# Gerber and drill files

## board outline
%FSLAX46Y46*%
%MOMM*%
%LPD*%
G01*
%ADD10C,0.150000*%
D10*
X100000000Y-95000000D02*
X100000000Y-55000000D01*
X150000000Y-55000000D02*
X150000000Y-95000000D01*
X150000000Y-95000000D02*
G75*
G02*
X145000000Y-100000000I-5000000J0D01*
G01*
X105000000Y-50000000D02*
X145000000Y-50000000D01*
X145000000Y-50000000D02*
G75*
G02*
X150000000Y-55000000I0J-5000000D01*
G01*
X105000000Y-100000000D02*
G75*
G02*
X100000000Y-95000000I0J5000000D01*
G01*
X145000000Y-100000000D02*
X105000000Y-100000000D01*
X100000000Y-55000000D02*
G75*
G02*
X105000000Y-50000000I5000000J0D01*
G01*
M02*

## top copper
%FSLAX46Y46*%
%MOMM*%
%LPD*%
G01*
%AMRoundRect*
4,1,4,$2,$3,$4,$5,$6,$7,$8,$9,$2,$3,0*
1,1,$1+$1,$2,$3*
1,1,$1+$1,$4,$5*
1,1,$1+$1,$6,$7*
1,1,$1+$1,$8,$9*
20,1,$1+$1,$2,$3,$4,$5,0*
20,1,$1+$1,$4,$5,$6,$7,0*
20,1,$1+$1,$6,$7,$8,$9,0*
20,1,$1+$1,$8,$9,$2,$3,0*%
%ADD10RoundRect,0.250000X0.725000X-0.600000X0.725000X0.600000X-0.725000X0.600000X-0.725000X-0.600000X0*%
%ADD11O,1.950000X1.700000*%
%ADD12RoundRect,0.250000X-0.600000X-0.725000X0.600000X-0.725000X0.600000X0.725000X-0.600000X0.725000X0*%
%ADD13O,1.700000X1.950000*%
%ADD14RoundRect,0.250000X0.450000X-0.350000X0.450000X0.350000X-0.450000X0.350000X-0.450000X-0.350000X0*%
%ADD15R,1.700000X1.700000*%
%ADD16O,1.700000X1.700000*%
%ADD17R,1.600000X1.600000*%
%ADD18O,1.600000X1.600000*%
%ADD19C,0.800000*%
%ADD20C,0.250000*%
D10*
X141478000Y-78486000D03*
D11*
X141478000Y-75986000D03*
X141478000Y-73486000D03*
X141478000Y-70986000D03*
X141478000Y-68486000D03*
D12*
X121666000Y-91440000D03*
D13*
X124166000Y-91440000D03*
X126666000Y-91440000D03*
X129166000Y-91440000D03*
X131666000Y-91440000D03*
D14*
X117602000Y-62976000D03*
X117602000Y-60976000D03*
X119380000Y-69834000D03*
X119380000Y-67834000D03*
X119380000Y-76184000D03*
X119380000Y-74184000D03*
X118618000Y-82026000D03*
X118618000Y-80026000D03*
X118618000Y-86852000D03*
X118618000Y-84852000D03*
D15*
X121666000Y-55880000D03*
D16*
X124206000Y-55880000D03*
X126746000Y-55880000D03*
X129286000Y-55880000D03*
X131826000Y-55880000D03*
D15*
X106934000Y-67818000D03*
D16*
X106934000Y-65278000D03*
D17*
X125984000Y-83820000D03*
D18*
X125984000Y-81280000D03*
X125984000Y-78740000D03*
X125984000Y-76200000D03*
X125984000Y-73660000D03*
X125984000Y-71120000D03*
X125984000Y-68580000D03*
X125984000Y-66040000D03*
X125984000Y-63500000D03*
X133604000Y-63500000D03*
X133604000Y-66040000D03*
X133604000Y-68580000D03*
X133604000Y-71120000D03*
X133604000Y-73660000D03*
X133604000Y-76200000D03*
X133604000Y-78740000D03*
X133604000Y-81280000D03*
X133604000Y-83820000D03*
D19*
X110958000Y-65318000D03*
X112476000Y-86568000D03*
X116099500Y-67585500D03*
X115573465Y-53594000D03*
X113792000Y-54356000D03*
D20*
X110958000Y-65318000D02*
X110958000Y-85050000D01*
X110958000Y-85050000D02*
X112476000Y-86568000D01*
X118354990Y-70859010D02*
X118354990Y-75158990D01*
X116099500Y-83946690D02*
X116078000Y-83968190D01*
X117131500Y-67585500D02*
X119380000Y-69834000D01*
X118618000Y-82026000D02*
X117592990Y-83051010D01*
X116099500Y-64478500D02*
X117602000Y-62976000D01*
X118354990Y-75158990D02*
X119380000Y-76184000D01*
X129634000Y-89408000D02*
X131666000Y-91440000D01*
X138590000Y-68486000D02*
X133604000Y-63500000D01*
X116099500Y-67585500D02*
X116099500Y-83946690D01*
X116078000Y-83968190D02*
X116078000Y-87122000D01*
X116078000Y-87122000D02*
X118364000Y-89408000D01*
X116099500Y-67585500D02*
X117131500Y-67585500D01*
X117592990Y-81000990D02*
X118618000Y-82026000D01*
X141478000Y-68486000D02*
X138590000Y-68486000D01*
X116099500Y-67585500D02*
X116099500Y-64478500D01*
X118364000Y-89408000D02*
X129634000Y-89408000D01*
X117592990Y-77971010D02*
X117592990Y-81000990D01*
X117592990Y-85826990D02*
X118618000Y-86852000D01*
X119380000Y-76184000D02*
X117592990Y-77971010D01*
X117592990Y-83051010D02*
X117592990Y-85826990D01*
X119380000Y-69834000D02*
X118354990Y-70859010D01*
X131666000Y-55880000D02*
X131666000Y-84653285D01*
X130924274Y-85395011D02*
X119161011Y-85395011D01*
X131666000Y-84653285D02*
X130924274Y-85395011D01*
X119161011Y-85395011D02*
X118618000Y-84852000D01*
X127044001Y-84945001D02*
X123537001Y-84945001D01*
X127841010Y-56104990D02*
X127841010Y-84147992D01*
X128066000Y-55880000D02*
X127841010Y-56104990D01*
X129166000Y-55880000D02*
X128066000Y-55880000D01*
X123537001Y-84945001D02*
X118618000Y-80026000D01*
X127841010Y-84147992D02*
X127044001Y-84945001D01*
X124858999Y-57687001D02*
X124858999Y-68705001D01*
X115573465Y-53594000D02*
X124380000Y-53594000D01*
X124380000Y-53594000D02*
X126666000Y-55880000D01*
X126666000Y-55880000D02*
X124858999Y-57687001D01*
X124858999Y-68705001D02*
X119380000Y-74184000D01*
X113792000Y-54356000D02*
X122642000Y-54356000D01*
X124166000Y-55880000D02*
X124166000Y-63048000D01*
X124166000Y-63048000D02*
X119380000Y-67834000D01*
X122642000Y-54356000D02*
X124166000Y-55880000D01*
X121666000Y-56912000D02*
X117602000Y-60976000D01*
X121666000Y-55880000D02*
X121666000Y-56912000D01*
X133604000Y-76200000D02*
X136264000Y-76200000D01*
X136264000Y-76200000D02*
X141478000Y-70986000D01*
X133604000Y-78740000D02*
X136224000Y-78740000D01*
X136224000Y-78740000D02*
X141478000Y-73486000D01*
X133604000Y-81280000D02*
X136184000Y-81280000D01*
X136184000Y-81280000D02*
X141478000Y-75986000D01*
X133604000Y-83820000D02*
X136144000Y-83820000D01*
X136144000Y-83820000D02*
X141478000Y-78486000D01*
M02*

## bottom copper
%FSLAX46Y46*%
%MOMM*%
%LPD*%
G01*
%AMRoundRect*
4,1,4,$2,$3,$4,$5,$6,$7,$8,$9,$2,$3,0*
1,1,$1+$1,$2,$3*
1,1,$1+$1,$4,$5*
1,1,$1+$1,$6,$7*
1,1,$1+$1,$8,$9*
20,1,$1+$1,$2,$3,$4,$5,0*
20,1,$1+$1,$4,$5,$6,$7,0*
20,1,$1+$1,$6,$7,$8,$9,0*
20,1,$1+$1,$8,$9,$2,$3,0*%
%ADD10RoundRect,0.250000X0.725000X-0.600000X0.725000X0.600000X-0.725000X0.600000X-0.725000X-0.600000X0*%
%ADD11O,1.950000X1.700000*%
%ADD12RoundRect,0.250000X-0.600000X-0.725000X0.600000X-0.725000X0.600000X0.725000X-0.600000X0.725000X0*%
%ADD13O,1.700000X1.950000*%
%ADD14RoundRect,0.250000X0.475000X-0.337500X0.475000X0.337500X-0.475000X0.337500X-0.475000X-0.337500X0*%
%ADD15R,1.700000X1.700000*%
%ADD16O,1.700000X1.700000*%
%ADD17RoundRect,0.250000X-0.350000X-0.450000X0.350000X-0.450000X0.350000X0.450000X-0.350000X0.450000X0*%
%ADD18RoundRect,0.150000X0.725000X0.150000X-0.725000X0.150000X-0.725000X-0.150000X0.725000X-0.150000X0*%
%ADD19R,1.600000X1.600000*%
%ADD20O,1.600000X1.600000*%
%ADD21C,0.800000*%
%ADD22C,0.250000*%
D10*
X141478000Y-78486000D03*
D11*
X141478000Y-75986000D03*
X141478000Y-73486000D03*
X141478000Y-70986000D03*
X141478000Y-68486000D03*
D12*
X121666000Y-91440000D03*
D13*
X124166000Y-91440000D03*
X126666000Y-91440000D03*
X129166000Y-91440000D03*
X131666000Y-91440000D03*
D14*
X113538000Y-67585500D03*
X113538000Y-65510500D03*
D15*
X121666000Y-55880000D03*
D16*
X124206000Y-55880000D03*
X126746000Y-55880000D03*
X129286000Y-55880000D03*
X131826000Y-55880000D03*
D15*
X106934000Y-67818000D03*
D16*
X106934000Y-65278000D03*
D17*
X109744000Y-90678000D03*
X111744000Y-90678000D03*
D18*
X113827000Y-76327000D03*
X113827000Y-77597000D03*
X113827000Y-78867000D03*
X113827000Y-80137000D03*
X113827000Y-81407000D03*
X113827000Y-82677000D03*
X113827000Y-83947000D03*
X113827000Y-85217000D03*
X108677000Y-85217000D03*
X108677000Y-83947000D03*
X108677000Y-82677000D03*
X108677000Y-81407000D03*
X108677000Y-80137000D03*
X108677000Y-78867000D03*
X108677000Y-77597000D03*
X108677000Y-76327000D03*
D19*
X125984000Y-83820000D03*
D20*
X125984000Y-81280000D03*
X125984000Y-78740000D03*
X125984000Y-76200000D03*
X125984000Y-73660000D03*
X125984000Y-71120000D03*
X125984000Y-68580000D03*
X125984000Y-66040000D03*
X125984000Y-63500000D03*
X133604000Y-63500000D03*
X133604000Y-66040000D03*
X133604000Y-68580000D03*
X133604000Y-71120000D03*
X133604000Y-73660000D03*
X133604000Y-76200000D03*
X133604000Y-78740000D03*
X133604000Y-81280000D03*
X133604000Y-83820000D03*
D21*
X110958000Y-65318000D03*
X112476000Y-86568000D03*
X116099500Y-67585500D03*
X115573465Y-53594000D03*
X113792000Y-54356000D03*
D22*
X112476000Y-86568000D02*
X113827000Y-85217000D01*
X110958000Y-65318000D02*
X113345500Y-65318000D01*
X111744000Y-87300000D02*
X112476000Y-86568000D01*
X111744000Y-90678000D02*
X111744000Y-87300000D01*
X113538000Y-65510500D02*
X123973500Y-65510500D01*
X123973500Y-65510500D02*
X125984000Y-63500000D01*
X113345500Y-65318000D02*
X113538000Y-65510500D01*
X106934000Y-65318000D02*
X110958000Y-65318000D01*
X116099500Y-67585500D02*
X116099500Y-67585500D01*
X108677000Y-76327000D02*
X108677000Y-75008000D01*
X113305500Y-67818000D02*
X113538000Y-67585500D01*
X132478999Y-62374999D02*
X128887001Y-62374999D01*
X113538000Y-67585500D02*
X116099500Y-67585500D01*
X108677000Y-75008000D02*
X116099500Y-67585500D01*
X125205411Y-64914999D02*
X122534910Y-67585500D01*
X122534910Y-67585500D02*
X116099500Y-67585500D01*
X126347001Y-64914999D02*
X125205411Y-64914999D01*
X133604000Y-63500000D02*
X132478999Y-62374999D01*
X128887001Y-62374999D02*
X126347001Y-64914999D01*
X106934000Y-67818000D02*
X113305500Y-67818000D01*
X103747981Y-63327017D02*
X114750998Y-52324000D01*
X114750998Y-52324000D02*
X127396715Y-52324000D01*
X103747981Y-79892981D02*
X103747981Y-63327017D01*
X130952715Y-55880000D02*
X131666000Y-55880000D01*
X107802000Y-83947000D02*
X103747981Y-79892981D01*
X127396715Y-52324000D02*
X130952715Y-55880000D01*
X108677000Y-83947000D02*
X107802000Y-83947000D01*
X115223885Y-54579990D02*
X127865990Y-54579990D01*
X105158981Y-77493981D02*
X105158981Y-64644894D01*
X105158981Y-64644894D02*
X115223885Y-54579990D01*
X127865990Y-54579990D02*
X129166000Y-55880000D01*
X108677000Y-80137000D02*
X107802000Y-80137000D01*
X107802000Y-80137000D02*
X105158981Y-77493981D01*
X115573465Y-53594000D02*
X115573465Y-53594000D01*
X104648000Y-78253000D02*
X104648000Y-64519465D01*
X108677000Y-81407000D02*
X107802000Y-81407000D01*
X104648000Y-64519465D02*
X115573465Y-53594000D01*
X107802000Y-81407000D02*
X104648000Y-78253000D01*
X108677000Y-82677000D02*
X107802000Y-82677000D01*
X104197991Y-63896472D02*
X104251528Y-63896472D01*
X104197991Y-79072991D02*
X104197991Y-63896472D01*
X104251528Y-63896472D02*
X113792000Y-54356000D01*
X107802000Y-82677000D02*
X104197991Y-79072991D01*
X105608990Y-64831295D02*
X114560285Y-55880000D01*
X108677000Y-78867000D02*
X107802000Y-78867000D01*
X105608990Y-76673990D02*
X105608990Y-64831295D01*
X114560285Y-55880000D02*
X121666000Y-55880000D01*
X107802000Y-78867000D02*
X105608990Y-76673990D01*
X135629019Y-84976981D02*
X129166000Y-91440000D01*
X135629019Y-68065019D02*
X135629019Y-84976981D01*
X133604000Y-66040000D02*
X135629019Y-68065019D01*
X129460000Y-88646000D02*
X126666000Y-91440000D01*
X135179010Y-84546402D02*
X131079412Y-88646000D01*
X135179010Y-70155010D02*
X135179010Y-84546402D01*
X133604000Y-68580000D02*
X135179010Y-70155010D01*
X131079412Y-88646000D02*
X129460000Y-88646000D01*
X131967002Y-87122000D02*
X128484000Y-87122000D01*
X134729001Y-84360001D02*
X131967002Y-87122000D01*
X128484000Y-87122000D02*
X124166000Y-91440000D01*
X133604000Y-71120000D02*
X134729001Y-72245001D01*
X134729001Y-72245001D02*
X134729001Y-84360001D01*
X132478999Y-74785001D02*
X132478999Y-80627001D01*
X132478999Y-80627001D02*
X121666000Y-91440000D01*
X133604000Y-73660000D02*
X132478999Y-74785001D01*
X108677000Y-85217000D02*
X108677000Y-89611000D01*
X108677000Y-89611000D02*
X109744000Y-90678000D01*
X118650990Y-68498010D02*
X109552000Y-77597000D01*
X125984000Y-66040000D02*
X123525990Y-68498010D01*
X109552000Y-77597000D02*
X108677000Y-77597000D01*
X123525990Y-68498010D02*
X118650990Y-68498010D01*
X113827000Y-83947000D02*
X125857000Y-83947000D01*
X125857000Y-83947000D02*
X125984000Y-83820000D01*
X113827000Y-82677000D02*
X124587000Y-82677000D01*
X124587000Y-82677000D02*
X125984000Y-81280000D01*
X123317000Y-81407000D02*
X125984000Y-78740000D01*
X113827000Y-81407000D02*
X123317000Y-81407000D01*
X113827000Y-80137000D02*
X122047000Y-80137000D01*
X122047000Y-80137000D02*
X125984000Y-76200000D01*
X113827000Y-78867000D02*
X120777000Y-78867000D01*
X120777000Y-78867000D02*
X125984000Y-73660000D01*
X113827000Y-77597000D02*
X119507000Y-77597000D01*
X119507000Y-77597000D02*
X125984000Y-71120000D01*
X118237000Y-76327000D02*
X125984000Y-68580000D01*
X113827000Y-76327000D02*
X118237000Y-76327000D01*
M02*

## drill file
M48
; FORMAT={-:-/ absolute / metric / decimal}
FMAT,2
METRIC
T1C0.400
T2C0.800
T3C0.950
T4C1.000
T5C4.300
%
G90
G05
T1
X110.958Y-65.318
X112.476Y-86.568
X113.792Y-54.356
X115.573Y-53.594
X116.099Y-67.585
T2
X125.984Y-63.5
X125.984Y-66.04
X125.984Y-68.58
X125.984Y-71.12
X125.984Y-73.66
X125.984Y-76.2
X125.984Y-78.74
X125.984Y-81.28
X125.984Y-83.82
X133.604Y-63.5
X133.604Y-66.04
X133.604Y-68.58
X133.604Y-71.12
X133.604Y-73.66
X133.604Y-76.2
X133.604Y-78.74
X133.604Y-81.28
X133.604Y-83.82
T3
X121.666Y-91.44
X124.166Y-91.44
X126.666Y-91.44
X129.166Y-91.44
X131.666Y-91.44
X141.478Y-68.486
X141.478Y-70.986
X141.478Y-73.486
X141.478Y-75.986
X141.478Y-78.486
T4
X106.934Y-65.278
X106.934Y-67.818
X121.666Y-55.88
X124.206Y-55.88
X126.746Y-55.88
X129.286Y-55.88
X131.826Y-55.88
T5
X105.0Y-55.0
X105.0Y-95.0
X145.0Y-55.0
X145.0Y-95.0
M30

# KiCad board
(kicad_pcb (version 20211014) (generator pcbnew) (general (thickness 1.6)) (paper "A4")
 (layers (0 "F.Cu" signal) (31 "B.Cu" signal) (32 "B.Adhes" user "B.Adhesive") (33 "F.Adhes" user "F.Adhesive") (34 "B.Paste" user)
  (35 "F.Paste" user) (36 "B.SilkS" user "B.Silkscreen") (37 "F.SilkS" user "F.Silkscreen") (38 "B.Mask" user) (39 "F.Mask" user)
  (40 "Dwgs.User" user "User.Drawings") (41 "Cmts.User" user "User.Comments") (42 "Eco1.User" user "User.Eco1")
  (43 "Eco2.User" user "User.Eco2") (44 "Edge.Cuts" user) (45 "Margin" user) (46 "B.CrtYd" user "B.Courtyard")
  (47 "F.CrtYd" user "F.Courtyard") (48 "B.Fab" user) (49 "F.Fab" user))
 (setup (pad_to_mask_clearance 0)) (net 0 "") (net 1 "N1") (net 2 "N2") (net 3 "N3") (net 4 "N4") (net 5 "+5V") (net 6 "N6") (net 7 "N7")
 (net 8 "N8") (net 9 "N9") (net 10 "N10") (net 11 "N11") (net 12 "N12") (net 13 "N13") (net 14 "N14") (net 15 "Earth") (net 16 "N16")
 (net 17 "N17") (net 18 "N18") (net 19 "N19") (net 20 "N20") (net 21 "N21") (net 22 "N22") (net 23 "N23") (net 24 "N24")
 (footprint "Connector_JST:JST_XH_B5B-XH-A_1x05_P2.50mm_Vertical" (layer "F.Cu") (at 141.478 78.486 90)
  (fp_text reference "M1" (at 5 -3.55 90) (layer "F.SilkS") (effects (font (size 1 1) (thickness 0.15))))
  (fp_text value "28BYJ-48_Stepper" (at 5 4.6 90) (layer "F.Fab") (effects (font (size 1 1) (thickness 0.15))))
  (pad "1" thru_hole roundrect locked (at 0 0 90) (size 1.7 1.95) (drill 0.95) (layers *.Cu *.Mask) (roundrect_rratio 0.1470588235)
   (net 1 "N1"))
  (pad "2" thru_hole oval locked (at 2.5 0 90) (size 1.7 1.95) (drill 0.95) (layers *.Cu *.Mask) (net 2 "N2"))
  (pad "3" thru_hole oval locked (at 5 0 90) (size 1.7 1.95) (drill 0.95) (layers *.Cu *.Mask) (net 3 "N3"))
  (pad "4" thru_hole oval locked (at 7.5 0 90) (size 1.7 1.95) (drill 0.95) (layers *.Cu *.Mask) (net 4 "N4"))
  (pad "5" thru_hole oval locked (at 10 0 90) (size 1.7 1.95) (drill 0.95) (layers *.Cu *.Mask) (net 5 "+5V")))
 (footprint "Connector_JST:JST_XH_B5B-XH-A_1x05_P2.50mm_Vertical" (layer "F.Cu") (at 121.666 91.44)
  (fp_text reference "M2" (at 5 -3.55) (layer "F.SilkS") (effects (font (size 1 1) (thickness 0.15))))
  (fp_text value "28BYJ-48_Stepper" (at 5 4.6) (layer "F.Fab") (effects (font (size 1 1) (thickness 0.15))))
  (pad "1" thru_hole roundrect locked (at 0 0) (size 1.7 1.95) (drill 0.95) (layers *.Cu *.Mask) (roundrect_rratio 0.1470588235)
   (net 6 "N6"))
  (pad "2" thru_hole oval locked (at 2.5 0) (size 1.7 1.95) (drill 0.95) (layers *.Cu *.Mask) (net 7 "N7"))
  (pad "3" thru_hole oval locked (at 5 0) (size 1.7 1.95) (drill 0.95) (layers *.Cu *.Mask) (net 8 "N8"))
  (pad "4" thru_hole oval locked (at 7.5 0) (size 1.7 1.95) (drill 0.95) (layers *.Cu *.Mask) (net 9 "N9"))
  (pad "5" thru_hole oval locked (at 10 0) (size 1.7 1.95) (drill 0.95) (layers *.Cu *.Mask) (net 5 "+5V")))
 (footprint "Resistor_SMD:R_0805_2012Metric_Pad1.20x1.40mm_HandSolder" (layer "F.Cu") (at 117.602 61.976 90)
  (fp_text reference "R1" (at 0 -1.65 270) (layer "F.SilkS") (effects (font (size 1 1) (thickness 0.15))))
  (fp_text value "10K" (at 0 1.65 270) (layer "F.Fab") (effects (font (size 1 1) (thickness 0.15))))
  (pad "1" smd roundrect locked (at -1 0 90) (size 1.2 1.4) (layers "F.Cu" "F.Paste" "F.Mask") (roundrect_rratio 0.2083333333) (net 5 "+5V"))
  (pad "2" smd roundrect locked (at 1 0 90) (size 1.2 1.4) (layers "F.Cu" "F.Paste" "F.Mask") (roundrect_rratio 0.2083333333) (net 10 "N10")))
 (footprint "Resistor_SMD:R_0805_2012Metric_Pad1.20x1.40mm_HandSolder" (layer "F.Cu") (at 119.38 68.834 90)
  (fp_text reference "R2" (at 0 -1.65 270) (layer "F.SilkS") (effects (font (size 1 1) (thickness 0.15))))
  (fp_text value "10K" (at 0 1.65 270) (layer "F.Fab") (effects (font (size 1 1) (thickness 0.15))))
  (pad "1" smd roundrect locked (at -1 0 90) (size 1.2 1.4) (layers "F.Cu" "F.Paste" "F.Mask") (roundrect_rratio 0.2083333333) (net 5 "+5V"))
  (pad "2" smd roundrect locked (at 1 0 90) (size 1.2 1.4) (layers "F.Cu" "F.Paste" "F.Mask") (roundrect_rratio 0.2083333333) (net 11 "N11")))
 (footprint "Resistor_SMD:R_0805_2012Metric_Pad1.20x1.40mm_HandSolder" (layer "F.Cu") (at 119.38 75.184 90)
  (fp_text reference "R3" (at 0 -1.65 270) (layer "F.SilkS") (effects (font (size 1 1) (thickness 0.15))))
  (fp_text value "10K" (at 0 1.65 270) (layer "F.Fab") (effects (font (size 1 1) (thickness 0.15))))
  (pad "1" smd roundrect locked (at -1 0 90) (size 1.2 1.4) (layers "F.Cu" "F.Paste" "F.Mask") (roundrect_rratio 0.2083333333) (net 5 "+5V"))
  (pad "2" smd roundrect locked (at 1 0 90) (size 1.2 1.4) (layers "F.Cu" "F.Paste" "F.Mask") (roundrect_rratio 0.2083333333) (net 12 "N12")))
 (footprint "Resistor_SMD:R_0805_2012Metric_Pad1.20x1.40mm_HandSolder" (layer "F.Cu") (at 118.618 81.026 90)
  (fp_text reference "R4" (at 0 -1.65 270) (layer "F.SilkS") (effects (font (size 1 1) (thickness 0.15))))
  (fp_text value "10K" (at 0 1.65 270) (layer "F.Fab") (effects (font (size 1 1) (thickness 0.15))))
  (pad "1" smd roundrect locked (at -1 0 90) (size 1.2 1.4) (layers "F.Cu" "F.Paste" "F.Mask") (roundrect_rratio 0.2083333333) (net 5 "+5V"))
  (pad "2" smd roundrect locked (at 1 0 90) (size 1.2 1.4) (layers "F.Cu" "F.Paste" "F.Mask") (roundrect_rratio 0.2083333333) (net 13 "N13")))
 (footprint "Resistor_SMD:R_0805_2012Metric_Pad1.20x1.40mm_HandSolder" (layer "F.Cu") (at 118.618 85.852 90)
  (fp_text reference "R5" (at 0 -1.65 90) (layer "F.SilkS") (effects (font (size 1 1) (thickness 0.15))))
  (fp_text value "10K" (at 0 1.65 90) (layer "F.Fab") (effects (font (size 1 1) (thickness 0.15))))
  (pad "1" smd roundrect locked (at -1 0 90) (size 1.2 1.4) (layers "F.Cu" "F.Paste" "F.Mask") (roundrect_rratio 0.2083333333) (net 5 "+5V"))
  (pad "2" smd roundrect locked (at 1 0 90) (size 1.2 1.4) (layers "F.Cu" "F.Paste" "F.Mask") (roundrect_rratio 0.2083333333) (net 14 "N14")))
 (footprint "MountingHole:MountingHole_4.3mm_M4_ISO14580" (layer "F.Cu") (at 105 55)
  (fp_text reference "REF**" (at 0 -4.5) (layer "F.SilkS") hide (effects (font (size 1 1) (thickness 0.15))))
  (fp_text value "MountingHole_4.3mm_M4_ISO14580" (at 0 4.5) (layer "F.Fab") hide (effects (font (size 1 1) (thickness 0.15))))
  (pad "" np_thru_hole circle locked (at 0 0) (size 4.3 4.3) (drill 4.3) (layers *.Cu *.Mask)))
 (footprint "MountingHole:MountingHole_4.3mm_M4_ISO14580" (layer "F.Cu") (at 145 55)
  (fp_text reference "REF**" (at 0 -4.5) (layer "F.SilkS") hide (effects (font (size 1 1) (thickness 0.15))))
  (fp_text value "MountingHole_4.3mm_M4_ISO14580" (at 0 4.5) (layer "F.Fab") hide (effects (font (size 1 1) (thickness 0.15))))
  (pad "" np_thru_hole circle locked (at 0 0) (size 4.3 4.3) (drill 4.3) (layers *.Cu *.Mask)))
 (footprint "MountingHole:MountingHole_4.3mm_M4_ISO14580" (layer "F.Cu") (at 105 95)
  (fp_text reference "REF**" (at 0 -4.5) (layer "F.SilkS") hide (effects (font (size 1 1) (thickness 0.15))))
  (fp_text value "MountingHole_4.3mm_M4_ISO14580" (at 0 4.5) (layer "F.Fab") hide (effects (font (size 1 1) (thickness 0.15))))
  (pad "" np_thru_hole circle locked (at 0 0) (size 4.3 4.3) (drill 4.3) (layers *.Cu *.Mask)))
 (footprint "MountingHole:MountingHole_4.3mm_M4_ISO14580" (layer "F.Cu") (at 145 95)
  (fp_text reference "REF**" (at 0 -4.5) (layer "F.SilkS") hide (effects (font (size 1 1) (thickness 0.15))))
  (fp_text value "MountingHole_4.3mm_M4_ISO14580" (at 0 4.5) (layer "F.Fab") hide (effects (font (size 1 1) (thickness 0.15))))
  (pad "" np_thru_hole circle locked (at 0 0) (size 4.3 4.3) (drill 4.3) (layers *.Cu *.Mask)))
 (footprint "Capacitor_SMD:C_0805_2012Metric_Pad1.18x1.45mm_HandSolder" (layer "B.Cu") (at 113.538 66.548 90)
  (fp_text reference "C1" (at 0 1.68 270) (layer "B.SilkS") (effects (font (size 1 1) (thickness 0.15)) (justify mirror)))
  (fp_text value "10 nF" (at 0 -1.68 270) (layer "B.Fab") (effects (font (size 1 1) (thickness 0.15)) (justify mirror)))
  (pad "1" smd roundrect locked (at -1.0375 0 90) (size 1.175 1.45) (layers "B.Cu" "B.Paste" "B.Mask") (roundrect_rratio 0.2127659574)
   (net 5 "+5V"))
  (pad "2" smd roundrect locked (at 1.0375 0 90) (size 1.175 1.45) (layers "B.Cu" "B.Paste" "B.Mask") (roundrect_rratio 0.2127659574)
   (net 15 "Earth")))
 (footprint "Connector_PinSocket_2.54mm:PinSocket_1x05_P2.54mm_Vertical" (layer "B.Cu") (at 121.666 55.88 -90)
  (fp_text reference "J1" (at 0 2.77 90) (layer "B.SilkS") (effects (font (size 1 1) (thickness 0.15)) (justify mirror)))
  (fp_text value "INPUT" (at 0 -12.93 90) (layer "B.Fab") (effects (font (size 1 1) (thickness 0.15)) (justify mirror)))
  (pad "1" thru_hole rect (at 0 0 270) (size 1.7 1.7) (drill 1) (layers *.Cu *.Mask) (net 10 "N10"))
  (pad "2" thru_hole oval (at 0 -2.54 270) (size 1.7 1.7) (drill 1) (layers *.Cu *.Mask) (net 11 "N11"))
  (pad "3" thru_hole oval (at 0 -5.08 270) (size 1.7 1.7) (drill 1) (layers *.Cu *.Mask) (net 12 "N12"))
  (pad "4" thru_hole oval (at 0 -7.62 270) (size 1.7 1.7) (drill 1) (layers *.Cu *.Mask) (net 13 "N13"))
  (pad "5" thru_hole oval (at 0 -10.16 270) (size 1.7 1.7) (drill 1) (layers *.Cu *.Mask) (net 14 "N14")))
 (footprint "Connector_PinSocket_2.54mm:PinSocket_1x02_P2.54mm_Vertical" (layer "B.Cu") (at 106.934 67.818)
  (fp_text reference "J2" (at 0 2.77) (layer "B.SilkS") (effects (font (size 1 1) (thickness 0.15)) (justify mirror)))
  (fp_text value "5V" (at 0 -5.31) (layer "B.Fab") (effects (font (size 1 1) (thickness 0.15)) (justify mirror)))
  (pad "1" thru_hole rect (at 0 0) (size 1.7 1.7) (drill 1) (layers *.Cu *.Mask) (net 5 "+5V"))
  (pad "2" thru_hole oval (at 0 -2.54) (size 1.7 1.7) (drill 1) (layers *.Cu *.Mask) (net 15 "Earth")))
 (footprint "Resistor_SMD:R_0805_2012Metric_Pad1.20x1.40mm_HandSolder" (layer "B.Cu") (at 110.744 90.678)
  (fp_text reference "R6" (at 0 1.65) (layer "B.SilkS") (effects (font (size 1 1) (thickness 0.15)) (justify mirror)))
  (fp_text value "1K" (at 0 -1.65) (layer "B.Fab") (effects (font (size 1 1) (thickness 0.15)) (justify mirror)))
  (pad "1" smd roundrect locked (at -1 0) (size 1.2 1.4) (layers "B.Cu" "B.Paste" "B.Mask") (roundrect_rratio 0.2083333333) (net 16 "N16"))
  (pad "2" smd roundrect locked (at 1 0) (size 1.2 1.4) (layers "B.Cu" "B.Paste" "B.Mask") (roundrect_rratio 0.2083333333) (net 15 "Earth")))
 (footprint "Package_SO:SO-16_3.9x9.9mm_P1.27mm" (layer "B.Cu") (at 111.252 80.772 180)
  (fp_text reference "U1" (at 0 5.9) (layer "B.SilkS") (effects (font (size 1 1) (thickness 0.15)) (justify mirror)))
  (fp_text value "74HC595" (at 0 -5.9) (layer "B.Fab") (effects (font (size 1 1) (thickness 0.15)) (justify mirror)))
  (pad "1" smd roundrect locked (at -2.575 4.445 180) (size 1.75 0.6) (layers "B.Cu" "B.Paste" "B.Mask") (roundrect_rratio 0.25)
   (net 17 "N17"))
  (pad "2" smd roundrect locked (at -2.575 3.175 180) (size 1.75 0.6) (layers "B.Cu" "B.Paste" "B.Mask") (roundrect_rratio 0.25)
   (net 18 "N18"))
  (pad "3" smd roundrect locked (at -2.575 1.905 180) (size 1.75 0.6) (layers "B.Cu" "B.Paste" "B.Mask") (roundrect_rratio 0.25)
   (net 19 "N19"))
  (pad "4" smd roundrect locked (at -2.575 0.635 180) (size 1.75 0.6) (layers "B.Cu" "B.Paste" "B.Mask") (roundrect_rratio 0.25)
   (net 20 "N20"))
  (pad "5" smd roundrect locked (at -2.575 -0.635 180) (size 1.75 0.6) (layers "B.Cu" "B.Paste" "B.Mask") (roundrect_rratio 0.25)
   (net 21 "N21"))
  (pad "6" smd roundrect locked (at -2.575 -1.905 180) (size 1.75 0.6) (layers "B.Cu" "B.Paste" "B.Mask") (roundrect_rratio 0.25)
   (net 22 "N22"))
  (pad "7" smd roundrect locked (at -2.575 -3.175 180) (size 1.75 0.6) (layers "B.Cu" "B.Paste" "B.Mask") (roundrect_rratio 0.25)
   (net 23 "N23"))
  (pad "8" smd roundrect locked (at -2.575 -4.445 180) (size 1.75 0.6) (layers "B.Cu" "B.Paste" "B.Mask") (roundrect_rratio 0.25)
   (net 15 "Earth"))
  (pad "9" smd roundrect locked (at 2.575 -4.445 180) (size 1.75 0.6) (layers "B.Cu" "B.Paste" "B.Mask") (roundrect_rratio 0.25)
   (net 16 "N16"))
  (pad "10" smd roundrect locked (at 2.575 -3.175 180) (size 1.75 0.6) (layers "B.Cu" "B.Paste" "B.Mask") (roundrect_rratio 0.25)
   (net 14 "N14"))
  (pad "11" smd roundrect locked (at 2.575 -1.905 180) (size 1.75 0.6) (layers "B.Cu" "B.Paste" "B.Mask") (roundrect_rratio 0.25)
   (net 11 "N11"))
  (pad "12" smd roundrect locked (at 2.575 -0.635 180) (size 1.75 0.6) (layers "B.Cu" "B.Paste" "B.Mask") (roundrect_rratio 0.25)
   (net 12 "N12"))
  (pad "13" smd roundrect locked (at 2.575 0.635 180) (size 1.75 0.6) (layers "B.Cu" "B.Paste" "B.Mask") (roundrect_rratio 0.25)
   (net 13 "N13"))
  (pad "14" smd roundrect locked (at 2.575 1.905 180) (size 1.75 0.6) (layers "B.Cu" "B.Paste" "B.Mask") (roundrect_rratio 0.25)
   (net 10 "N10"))
  (pad "15" smd roundrect locked (at 2.575 3.175 180) (size 1.75 0.6) (layers "B.Cu" "B.Paste" "B.Mask") (roundrect_rratio 0.25)
   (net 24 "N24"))
  (pad "16" smd roundrect locked (at 2.575 4.445 180) (size 1.75 0.6) (layers "B.Cu" "B.Paste" "B.Mask") (roundrect_rratio 0.25)
   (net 5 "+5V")))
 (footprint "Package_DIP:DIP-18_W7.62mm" (layer "B.Cu") (at 125.984 83.82)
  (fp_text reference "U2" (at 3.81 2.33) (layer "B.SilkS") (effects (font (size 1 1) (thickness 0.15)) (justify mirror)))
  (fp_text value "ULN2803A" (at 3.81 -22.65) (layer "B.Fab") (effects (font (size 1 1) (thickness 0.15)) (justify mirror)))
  (pad "1" thru_hole rect locked (at 0 0) (size 1.6 1.6) (drill 0.8) (layers *.Cu *.Mask) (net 23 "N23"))
  (pad "2" thru_hole oval locked (at 0 -2.54) (size 1.6 1.6) (drill 0.8) (layers *.Cu *.Mask) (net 22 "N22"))
  (pad "3" thru_hole oval locked (at 0 -5.08) (size 1.6 1.6) (drill 0.8) (layers *.Cu *.Mask) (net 21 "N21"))
  (pad "4" thru_hole oval locked (at 0 -7.62) (size 1.6 1.6) (drill 0.8) (layers *.Cu *.Mask) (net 20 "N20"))
  (pad "5" thru_hole oval locked (at 0 -10.16) (size 1.6 1.6) (drill 0.8) (layers *.Cu *.Mask) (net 19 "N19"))
  (pad "6" thru_hole oval locked (at 0 -12.7) (size 1.6 1.6) (drill 0.8) (layers *.Cu *.Mask) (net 18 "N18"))
  (pad "7" thru_hole oval locked (at 0 -15.24) (size 1.6 1.6) (drill 0.8) (layers *.Cu *.Mask) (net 17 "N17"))
  (pad "8" thru_hole oval locked (at 0 -17.78) (size 1.6 1.6) (drill 0.8) (layers *.Cu *.Mask) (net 24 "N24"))
  (pad "9" thru_hole oval locked (at 0 -20.32) (size 1.6 1.6) (drill 0.8) (layers *.Cu *.Mask) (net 15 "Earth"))
  (pad "10" thru_hole oval locked (at 7.62 -20.32) (size 1.6 1.6) (drill 0.8) (layers *.Cu *.Mask) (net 5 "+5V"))
  (pad "11" thru_hole oval locked (at 7.62 -17.78) (size 1.6 1.6) (drill 0.8) (layers *.Cu *.Mask) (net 9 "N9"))
  (pad "12" thru_hole oval locked (at 7.62 -15.24) (size 1.6 1.6) (drill 0.8) (layers *.Cu *.Mask) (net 8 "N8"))
  (pad "13" thru_hole oval locked (at 7.62 -12.7) (size 1.6 1.6) (drill 0.8) (layers *.Cu *.Mask) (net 7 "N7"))
  (pad "14" thru_hole oval locked (at 7.62 -10.16) (size 1.6 1.6) (drill 0.8) (layers *.Cu *.Mask) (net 6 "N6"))
  (pad "15" thru_hole oval locked (at 7.62 -7.62) (size 1.6 1.6) (drill 0.8) (layers *.Cu *.Mask) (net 4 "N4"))
  (pad "16" thru_hole oval locked (at 7.62 -5.08) (size 1.6 1.6) (drill 0.8) (layers *.Cu *.Mask) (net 3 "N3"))
  (pad "17" thru_hole oval locked (at 7.62 -2.54) (size 1.6 1.6) (drill 0.8) (layers *.Cu *.Mask) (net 2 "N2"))
  (pad "18" thru_hole oval locked (at 7.62 0) (size 1.6 1.6) (drill 0.8) (layers *.Cu *.Mask) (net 1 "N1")))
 (gr_line (start 100 95) (end 100 55) (layer "Edge.Cuts") (width 0.15))
 (gr_line (start 150 55) (end 150 95) (layer "Edge.Cuts") (width 0.15))
 (gr_arc (start 150 95) (mid 148.535534 98.535534) (end 145 100) (layer "Edge.Cuts") (width 0.15))
 (gr_line (start 105 50) (end 145 50) (layer "Edge.Cuts") (width 0.15))
 (gr_arc (start 145 50) (mid 148.535534 51.464466) (end 150 55) (layer "Edge.Cuts") (width 0.15))
 (gr_arc (start 105 100) (mid 101.464466 98.535534) (end 100 95) (layer "Edge.Cuts") (width 0.15))
 (gr_line (start 145 100) (end 105 100) (layer "Edge.Cuts") (width 0.15))
 (gr_arc (start 100 55) (mid 101.464466 51.464466) (end 105 50) (layer "Edge.Cuts") (width 0.15))
 (segment (start 110.958 65.318) (end 110.958 85.05) (width 0.25) (layer "F.Cu") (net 15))
 (segment (start 110.958 85.05) (end 112.476 86.568) (width 0.25) (layer "F.Cu") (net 15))
 (via (at 110.958 65.318) (size 0.8) (drill 0.4) (layers "F.Cu" "B.Cu") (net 15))
 (via (at 112.476 86.568) (size 0.8) (drill 0.4) (layers "F.Cu" "B.Cu") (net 15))
 (segment (start 112.476 86.568) (end 113.827 85.217) (width 0.25) (layer "B.Cu") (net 15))
 (segment (start 110.958 65.318) (end 113.3455 65.318) (width 0.25) (layer "B.Cu") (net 15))
 (segment (start 111.744 87.3) (end 112.476 86.568) (width 0.25) (layer "B.Cu") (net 15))
 (segment (start 111.744 90.678) (end 111.744 87.3) (width 0.25) (layer "B.Cu") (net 15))
 (segment (start 113.538 65.5105) (end 123.9735 65.5105) (width 0.25) (layer "B.Cu") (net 15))
 (segment (start 123.9735 65.5105) (end 125.984 63.5) (width 0.25) (layer "B.Cu") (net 15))
 (segment (start 113.3455 65.318) (end 113.538 65.5105) (width 0.25) (layer "B.Cu") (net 15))
 (segment (start 106.934 65.318) (end 110.958 65.318) (width 0.25) (layer "B.Cu") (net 15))
 (segment (start 118.35499 70.85901) (end 118.35499 75.15899) (width 0.25) (layer "F.Cu") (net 5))
 (segment (start 116.0995 83.94669) (end 116.078 83.96819) (width 0.25) (layer "F.Cu") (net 5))
 (segment (start 117.1315 67.5855) (end 119.38 69.834) (width 0.25) (layer "F.Cu") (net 5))
 (segment (start 118.618 82.026) (end 117.59299 83.05101) (width 0.25) (layer "F.Cu") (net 5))
 (segment (start 116.0995 64.4785) (end 117.602 62.976) (width 0.25) (layer "F.Cu") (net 5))
 (segment (start 118.35499 75.15899) (end 119.38 76.184) (width 0.25) (layer "F.Cu") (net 5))
 (segment (start 129.634 89.408) (end 131.666 91.44) (width 0.25) (layer "F.Cu") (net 5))
 (segment (start 138.59 68.486) (end 133.604 63.5) (width 0.25) (layer "F.Cu") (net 5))
 (segment (start 116.0995 67.5855) (end 116.0995 83.94669) (width 0.25) (layer "F.Cu") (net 5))
 (segment (start 116.078 83.96819) (end 116.078 87.122) (width 0.25) (layer "F.Cu") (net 5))
 (segment (start 116.078 87.122) (end 118.364 89.408) (width 0.25) (layer "F.Cu") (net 5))
 (segment (start 116.0995 67.5855) (end 117.1315 67.5855) (width 0.25) (layer "F.Cu") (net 5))
 (segment (start 117.59299 81.00099) (end 118.618 82.026) (width 0.25) (layer "F.Cu") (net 5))
 (segment (start 141.478 68.486) (end 138.59 68.486) (width 0.25) (layer "F.Cu") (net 5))
 (segment (start 116.0995 67.5855) (end 116.0995 64.4785) (width 0.25) (layer "F.Cu") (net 5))
 (segment (start 118.364 89.408) (end 129.634 89.408) (width 0.25) (layer "F.Cu") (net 5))
 (segment (start 117.59299 77.97101) (end 117.59299 81.00099) (width 0.25) (layer "F.Cu") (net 5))
 (segment (start 117.59299 85.82699) (end 118.618 86.852) (width 0.25) (layer "F.Cu") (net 5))
 (segment (start 119.38 76.184) (end 117.59299 77.97101) (width 0.25) (layer "F.Cu") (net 5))
 (segment (start 117.59299 83.05101) (end 117.59299 85.82699) (width 0.25) (layer "F.Cu") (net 5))
 (segment (start 119.38 69.834) (end 118.35499 70.85901) (width 0.25) (layer "F.Cu") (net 5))
 (via (at 116.0995 67.5855) (size 0.8) (drill 0.4) (layers "F.Cu" "B.Cu") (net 5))
 (segment (start 116.0995 67.5855) (end 116.0995 67.5855) (width 0.25) (layer "B.Cu") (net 5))
 (segment (start 108.677 76.327) (end 108.677 75.008) (width 0.25) (layer "B.Cu") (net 5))
 (segment (start 113.3055 67.818) (end 113.538 67.5855) (width 0.25) (layer "B.Cu") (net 5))
 (segment (start 132.478999 62.374999) (end 128.887001 62.374999) (width 0.25) (layer "B.Cu") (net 5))
 (segment (start 113.538 67.5855) (end 116.0995 67.5855) (width 0.25) (layer "B.Cu") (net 5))
 (segment (start 108.677 75.008) (end 116.0995 67.5855) (width 0.25) (layer "B.Cu") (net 5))
 (segment (start 125.205411 64.914999) (end 122.53491 67.5855) (width 0.25) (layer "B.Cu") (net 5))
 (segment (start 122.53491 67.5855) (end 116.0995 67.5855) (width 0.25) (layer "B.Cu") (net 5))
 (segment (start 126.347001 64.914999) (end 125.205411 64.914999) (width 0.25) (layer "B.Cu") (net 5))
 (segment (start 133.604 63.5) (end 132.478999 62.374999) (width 0.25) (layer "B.Cu") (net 5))
 (segment (start 128.887001 62.374999) (end 126.347001 64.914999) (width 0.25) (layer "B.Cu") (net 5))
 (segment (start 106.934 67.818) (end 113.3055 67.818) (width 0.25) (layer "B.Cu") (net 5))
 (segment (start 131.666 55.88) (end 131.666 84.653285) (width 0.25) (layer "F.Cu") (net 14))
 (segment (start 130.924274 85.395011) (end 119.161011 85.395011) (width 0.25) (layer "F.Cu") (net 14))
 (segment (start 131.666 84.653285) (end 130.924274 85.395011) (width 0.25) (layer "F.Cu") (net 14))
 (segment (start 119.161011 85.395011) (end 118.618 84.852) (width 0.25) (layer "F.Cu") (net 14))
 (segment (start 103.747981 63.327017) (end 114.750998 52.324) (width 0.25) (layer "B.Cu") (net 14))
 (segment (start 114.750998 52.324) (end 127.396715 52.324) (width 0.25) (layer "B.Cu") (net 14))
 (segment (start 103.747981 79.892981) (end 103.747981 63.327017) (width 0.25) (layer "B.Cu") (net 14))
 (segment (start 130.952715 55.88) (end 131.666 55.88) (width 0.25) (layer "B.Cu") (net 14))
 (segment (start 107.802 83.947) (end 103.747981 79.892981) (width 0.25) (layer "B.Cu") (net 14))
 (segment (start 127.396715 52.324) (end 130.952715 55.88) (width 0.25) (layer "B.Cu") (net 14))
 (segment (start 108.677 83.947) (end 107.802 83.947) (width 0.25) (layer "B.Cu") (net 14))
 (segment (start 127.044001 84.945001) (end 123.537001 84.945001) (width 0.25) (layer "F.Cu") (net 13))
 (segment (start 127.84101 56.10499) (end 127.84101 84.147992) (width 0.25) (layer "F.Cu") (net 13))
 (segment (start 128.066 55.88) (end 127.84101 56.10499) (width 0.25) (layer "F.Cu") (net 13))
 (segment (start 129.166 55.88) (end 128.066 55.88) (width 0.25) (layer "F.Cu") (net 13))
 (segment (start 123.537001 84.945001) (end 118.618 80.026) (width 0.25) (layer "F.Cu") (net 13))
 (segment (start 127.84101 84.147992) (end 127.044001 84.945001) (width 0.25) (layer "F.Cu") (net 13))
 (segment (start 115.223885 54.57999) (end 127.86599 54.57999) (width 0.25) (layer "B.Cu") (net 13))
 (segment (start 105.158981 77.493981) (end 105.158981 64.644894) (width 0.25) (layer "B.Cu") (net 13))
 (segment (start 105.158981 64.644894) (end 115.223885 54.57999) (width 0.25) (layer "B.Cu") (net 13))
 (segment (start 127.86599 54.57999) (end 129.166 55.88) (width 0.25) (layer "B.Cu") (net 13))
 (segment (start 108.677 80.137) (end 107.802 80.137) (width 0.25) (layer "B.Cu") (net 13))
 (segment (start 107.802 80.137) (end 105.158981 77.493981) (width 0.25) (layer "B.Cu") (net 13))
 (segment (start 124.858999 57.687001) (end 124.858999 68.705001) (width 0.25) (layer "F.Cu") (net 12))
 (segment (start 115.573465 53.594) (end 124.38 53.594) (width 0.25) (layer "F.Cu") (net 12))
 (segment (start 124.38 53.594) (end 126.666 55.88) (width 0.25) (layer "F.Cu") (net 12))
 (segment (start 126.666 55.88) (end 124.858999 57.687001) (width 0.25) (layer "F.Cu") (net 12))
 (segment (start 124.858999 68.705001) (end 119.38 74.184) (width 0.25) (layer "F.Cu") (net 12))
 (via (at 115.573465 53.594) (size 0.8) (drill 0.4) (layers "F.Cu" "B.Cu") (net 12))
 (segment (start 115.573465 53.594) (end 115.573465 53.594) (width 0.25) (layer "B.Cu") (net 12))
 (segment (start 104.648 78.253) (end 104.648 64.519465) (width 0.25) (layer "B.Cu") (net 12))
 (segment (start 108.677 81.407) (end 107.802 81.407) (width 0.25) (layer "B.Cu") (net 12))
 (segment (start 104.648 64.519465) (end 115.573465 53.594) (width 0.25) (layer "B.Cu") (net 12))
 (segment (start 107.802 81.407) (end 104.648 78.253) (width 0.25) (layer "B.Cu") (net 12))
 (segment (start 113.792 54.356) (end 122.642 54.356) (width 0.25) (layer "F.Cu") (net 11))
 (segment (start 124.166 55.88) (end 124.166 63.048) (width 0.25) (layer "F.Cu") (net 11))
 (segment (start 124.166 63.048) (end 119.38 67.834) (width 0.25) (layer "F.Cu") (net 11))
 (segment (start 122.642 54.356) (end 124.166 55.88) (width 0.25) (layer "F.Cu") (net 11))
 (via (at 113.792 54.356) (size 0.8) (drill 0.4) (layers "F.Cu" "B.Cu") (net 11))
 (segment (start 108.677 82.677) (end 107.802 82.677) (width 0.25) (layer "B.Cu") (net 11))
 (segment (start 104.197991 63.896472) (end 104.251528 63.896472) (width 0.25) (layer "B.Cu") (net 11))
 (segment (start 104.197991 79.072991) (end 104.197991 63.896472) (width 0.25) (layer "B.Cu") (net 11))
 (segment (start 104.251528 63.896472) (end 113.792 54.356) (width 0.25) (layer "B.Cu") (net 11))
 (segment (start 107.802 82.677) (end 104.197991 79.072991) (width 0.25) (layer "B.Cu") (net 11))
 (segment (start 121.666 56.912) (end 117.602 60.976) (width 0.25) (layer "F.Cu") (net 10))
 (segment (start 121.666 55.88) (end 121.666 56.912) (width 0.25) (layer "F.Cu") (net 10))
 (segment (start 105.60899 64.831295) (end 114.560285 55.88) (width 0.25) (layer "B.Cu") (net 10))
 (segment (start 108.677 78.867) (end 107.802 78.867) (width 0.25) (layer "B.Cu") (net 10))
 (segment (start 105.60899 76.67399) (end 105.60899 64.831295) (width 0.25) (layer "B.Cu") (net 10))
 (segment (start 114.560285 55.88) (end 121.666 55.88) (width 0.25) (layer "B.Cu") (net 10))
 (segment (start 107.802 78.867) (end 105.60899 76.67399) (width 0.25) (layer "B.Cu") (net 10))
 (segment (start 133.604 76.2) (end 136.264 76.2) (width 0.25) (layer "F.Cu") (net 4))
 (segment (start 136.264 76.2) (end 141.478 70.986) (width 0.25) (layer "F.Cu") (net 4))
 (segment (start 133.604 78.74) (end 136.224 78.74) (width 0.25) (layer "F.Cu") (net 3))
 (segment (start 136.224 78.74) (end 141.478 73.486) (width 0.25) (layer "F.Cu") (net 3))
 (segment (start 133.604 81.28) (end 136.184 81.28) (width 0.25) (layer "F.Cu") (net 2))
 (segment (start 136.184 81.28) (end 141.478 75.986) (width 0.25) (layer "F.Cu") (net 2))
 (segment (start 133.604 83.82) (end 136.144 83.82) (width 0.25) (layer "F.Cu") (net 1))
 (segment (start 136.144 83.82) (end 141.478 78.486) (width 0.25) (layer "F.Cu") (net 1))
 (segment (start 135.629019 84.976981) (end 129.166 91.44) (width 0.25) (layer "B.Cu") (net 9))
 (segment (start 135.629019 68.065019) (end 135.629019 84.976981) (width 0.25) (layer "B.Cu") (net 9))
 (segment (start 133.604 66.04) (end 135.629019 68.065019) (width 0.25) (layer "B.Cu") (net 9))
 (segment (start 129.46 88.646) (end 126.666 91.44) (width 0.25) (layer "B.Cu") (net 8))
 (segment (start 135.17901 84.546402) (end 131.079412 88.646) (width 0.25) (layer "B.Cu") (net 8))
 (segment (start 135.17901 70.15501) (end 135.17901 84.546402) (width 0.25) (layer "B.Cu") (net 8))
 (segment (start 133.604 68.58) (end 135.17901 70.15501) (width 0.25) (layer "B.Cu") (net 8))
 (segment (start 131.079412 88.646) (end 129.46 88.646) (width 0.25) (layer "B.Cu") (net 8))
 (segment (start 131.967002 87.122) (end 128.484 87.122) (width 0.25) (layer "B.Cu") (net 7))
 (segment (start 134.729001 84.360001) (end 131.967002 87.122) (width 0.25) (layer "B.Cu") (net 7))
 (segment (start 128.484 87.122) (end 124.166 91.44) (width 0.25) (layer "B.Cu") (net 7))
 (segment (start 133.604 71.12) (end 134.729001 72.245001) (width 0.25) (layer "B.Cu") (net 7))
 (segment (start 134.729001 72.245001) (end 134.729001 84.360001) (width 0.25) (layer "B.Cu") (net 7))
 (segment (start 132.478999 74.785001) (end 132.478999 80.627001) (width 0.25) (layer "B.Cu") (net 6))
 (segment (start 132.478999 80.627001) (end 121.666 91.44) (width 0.25) (layer "B.Cu") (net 6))
 (segment (start 133.604 73.66) (end 132.478999 74.785001) (width 0.25) (layer "B.Cu") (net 6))
 (segment (start 108.677 85.217) (end 108.677 89.611) (width 0.25) (layer "B.Cu") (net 16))
 (segment (start 108.677 89.611) (end 109.744 90.678) (width 0.25) (layer "B.Cu") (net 16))
 (segment (start 118.65099 68.49801) (end 109.552 77.597) (width 0.25) (layer "B.Cu") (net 24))
 (segment (start 125.984 66.04) (end 123.52599 68.49801) (width 0.25) (layer "B.Cu") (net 24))
 (segment (start 109.552 77.597) (end 108.677 77.597) (width 0.25) (layer "B.Cu") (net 24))
 (segment (start 123.52599 68.49801) (end 118.65099 68.49801) (width 0.25) (layer "B.Cu") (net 24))
 (segment (start 113.827 83.947) (end 125.857 83.947) (width 0.25) (layer "B.Cu") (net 23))
 (segment (start 125.857 83.947) (end 125.984 83.82) (width 0.25) (layer "B.Cu") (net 23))
 (segment (start 113.827 82.677) (end 124.587 82.677) (width 0.25) (layer "B.Cu") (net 22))
 (segment (start 124.587 82.677) (end 125.984 81.28) (width 0.25) (layer "B.Cu") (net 22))
 (segment (start 123.317 81.407) (end 125.984 78.74) (width 0.25) (layer "B.Cu") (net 21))
 (segment (start 113.827 81.407) (end 123.317 81.407) (width 0.25) (layer "B.Cu") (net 21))
 (segment (start 113.827 80.137) (end 122.047 80.137) (width 0.25) (layer "B.Cu") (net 20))
 (segment (start 122.047 80.137) (end 125.984 76.2) (width 0.25) (layer "B.Cu") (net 20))
 (segment (start 113.827 78.867) (end 120.777 78.867) (width 0.25) (layer "B.Cu") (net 19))
 (segment (start 120.777 78.867) (end 125.984 73.66) (width 0.25) (layer "B.Cu") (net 19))
 (segment (start 113.827 77.597) (end 119.507 77.597) (width 0.25) (layer "B.Cu") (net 18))
 (segment (start 119.507 77.597) (end 125.984 71.12) (width 0.25) (layer "B.Cu") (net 18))
 (segment (start 118.237 76.327) (end 125.984 68.58) (width 0.25) (layer "B.Cu") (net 17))
 (segment (start 113.827 76.327) (end 118.237 76.327) (width 0.25) (layer "B.Cu") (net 17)))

